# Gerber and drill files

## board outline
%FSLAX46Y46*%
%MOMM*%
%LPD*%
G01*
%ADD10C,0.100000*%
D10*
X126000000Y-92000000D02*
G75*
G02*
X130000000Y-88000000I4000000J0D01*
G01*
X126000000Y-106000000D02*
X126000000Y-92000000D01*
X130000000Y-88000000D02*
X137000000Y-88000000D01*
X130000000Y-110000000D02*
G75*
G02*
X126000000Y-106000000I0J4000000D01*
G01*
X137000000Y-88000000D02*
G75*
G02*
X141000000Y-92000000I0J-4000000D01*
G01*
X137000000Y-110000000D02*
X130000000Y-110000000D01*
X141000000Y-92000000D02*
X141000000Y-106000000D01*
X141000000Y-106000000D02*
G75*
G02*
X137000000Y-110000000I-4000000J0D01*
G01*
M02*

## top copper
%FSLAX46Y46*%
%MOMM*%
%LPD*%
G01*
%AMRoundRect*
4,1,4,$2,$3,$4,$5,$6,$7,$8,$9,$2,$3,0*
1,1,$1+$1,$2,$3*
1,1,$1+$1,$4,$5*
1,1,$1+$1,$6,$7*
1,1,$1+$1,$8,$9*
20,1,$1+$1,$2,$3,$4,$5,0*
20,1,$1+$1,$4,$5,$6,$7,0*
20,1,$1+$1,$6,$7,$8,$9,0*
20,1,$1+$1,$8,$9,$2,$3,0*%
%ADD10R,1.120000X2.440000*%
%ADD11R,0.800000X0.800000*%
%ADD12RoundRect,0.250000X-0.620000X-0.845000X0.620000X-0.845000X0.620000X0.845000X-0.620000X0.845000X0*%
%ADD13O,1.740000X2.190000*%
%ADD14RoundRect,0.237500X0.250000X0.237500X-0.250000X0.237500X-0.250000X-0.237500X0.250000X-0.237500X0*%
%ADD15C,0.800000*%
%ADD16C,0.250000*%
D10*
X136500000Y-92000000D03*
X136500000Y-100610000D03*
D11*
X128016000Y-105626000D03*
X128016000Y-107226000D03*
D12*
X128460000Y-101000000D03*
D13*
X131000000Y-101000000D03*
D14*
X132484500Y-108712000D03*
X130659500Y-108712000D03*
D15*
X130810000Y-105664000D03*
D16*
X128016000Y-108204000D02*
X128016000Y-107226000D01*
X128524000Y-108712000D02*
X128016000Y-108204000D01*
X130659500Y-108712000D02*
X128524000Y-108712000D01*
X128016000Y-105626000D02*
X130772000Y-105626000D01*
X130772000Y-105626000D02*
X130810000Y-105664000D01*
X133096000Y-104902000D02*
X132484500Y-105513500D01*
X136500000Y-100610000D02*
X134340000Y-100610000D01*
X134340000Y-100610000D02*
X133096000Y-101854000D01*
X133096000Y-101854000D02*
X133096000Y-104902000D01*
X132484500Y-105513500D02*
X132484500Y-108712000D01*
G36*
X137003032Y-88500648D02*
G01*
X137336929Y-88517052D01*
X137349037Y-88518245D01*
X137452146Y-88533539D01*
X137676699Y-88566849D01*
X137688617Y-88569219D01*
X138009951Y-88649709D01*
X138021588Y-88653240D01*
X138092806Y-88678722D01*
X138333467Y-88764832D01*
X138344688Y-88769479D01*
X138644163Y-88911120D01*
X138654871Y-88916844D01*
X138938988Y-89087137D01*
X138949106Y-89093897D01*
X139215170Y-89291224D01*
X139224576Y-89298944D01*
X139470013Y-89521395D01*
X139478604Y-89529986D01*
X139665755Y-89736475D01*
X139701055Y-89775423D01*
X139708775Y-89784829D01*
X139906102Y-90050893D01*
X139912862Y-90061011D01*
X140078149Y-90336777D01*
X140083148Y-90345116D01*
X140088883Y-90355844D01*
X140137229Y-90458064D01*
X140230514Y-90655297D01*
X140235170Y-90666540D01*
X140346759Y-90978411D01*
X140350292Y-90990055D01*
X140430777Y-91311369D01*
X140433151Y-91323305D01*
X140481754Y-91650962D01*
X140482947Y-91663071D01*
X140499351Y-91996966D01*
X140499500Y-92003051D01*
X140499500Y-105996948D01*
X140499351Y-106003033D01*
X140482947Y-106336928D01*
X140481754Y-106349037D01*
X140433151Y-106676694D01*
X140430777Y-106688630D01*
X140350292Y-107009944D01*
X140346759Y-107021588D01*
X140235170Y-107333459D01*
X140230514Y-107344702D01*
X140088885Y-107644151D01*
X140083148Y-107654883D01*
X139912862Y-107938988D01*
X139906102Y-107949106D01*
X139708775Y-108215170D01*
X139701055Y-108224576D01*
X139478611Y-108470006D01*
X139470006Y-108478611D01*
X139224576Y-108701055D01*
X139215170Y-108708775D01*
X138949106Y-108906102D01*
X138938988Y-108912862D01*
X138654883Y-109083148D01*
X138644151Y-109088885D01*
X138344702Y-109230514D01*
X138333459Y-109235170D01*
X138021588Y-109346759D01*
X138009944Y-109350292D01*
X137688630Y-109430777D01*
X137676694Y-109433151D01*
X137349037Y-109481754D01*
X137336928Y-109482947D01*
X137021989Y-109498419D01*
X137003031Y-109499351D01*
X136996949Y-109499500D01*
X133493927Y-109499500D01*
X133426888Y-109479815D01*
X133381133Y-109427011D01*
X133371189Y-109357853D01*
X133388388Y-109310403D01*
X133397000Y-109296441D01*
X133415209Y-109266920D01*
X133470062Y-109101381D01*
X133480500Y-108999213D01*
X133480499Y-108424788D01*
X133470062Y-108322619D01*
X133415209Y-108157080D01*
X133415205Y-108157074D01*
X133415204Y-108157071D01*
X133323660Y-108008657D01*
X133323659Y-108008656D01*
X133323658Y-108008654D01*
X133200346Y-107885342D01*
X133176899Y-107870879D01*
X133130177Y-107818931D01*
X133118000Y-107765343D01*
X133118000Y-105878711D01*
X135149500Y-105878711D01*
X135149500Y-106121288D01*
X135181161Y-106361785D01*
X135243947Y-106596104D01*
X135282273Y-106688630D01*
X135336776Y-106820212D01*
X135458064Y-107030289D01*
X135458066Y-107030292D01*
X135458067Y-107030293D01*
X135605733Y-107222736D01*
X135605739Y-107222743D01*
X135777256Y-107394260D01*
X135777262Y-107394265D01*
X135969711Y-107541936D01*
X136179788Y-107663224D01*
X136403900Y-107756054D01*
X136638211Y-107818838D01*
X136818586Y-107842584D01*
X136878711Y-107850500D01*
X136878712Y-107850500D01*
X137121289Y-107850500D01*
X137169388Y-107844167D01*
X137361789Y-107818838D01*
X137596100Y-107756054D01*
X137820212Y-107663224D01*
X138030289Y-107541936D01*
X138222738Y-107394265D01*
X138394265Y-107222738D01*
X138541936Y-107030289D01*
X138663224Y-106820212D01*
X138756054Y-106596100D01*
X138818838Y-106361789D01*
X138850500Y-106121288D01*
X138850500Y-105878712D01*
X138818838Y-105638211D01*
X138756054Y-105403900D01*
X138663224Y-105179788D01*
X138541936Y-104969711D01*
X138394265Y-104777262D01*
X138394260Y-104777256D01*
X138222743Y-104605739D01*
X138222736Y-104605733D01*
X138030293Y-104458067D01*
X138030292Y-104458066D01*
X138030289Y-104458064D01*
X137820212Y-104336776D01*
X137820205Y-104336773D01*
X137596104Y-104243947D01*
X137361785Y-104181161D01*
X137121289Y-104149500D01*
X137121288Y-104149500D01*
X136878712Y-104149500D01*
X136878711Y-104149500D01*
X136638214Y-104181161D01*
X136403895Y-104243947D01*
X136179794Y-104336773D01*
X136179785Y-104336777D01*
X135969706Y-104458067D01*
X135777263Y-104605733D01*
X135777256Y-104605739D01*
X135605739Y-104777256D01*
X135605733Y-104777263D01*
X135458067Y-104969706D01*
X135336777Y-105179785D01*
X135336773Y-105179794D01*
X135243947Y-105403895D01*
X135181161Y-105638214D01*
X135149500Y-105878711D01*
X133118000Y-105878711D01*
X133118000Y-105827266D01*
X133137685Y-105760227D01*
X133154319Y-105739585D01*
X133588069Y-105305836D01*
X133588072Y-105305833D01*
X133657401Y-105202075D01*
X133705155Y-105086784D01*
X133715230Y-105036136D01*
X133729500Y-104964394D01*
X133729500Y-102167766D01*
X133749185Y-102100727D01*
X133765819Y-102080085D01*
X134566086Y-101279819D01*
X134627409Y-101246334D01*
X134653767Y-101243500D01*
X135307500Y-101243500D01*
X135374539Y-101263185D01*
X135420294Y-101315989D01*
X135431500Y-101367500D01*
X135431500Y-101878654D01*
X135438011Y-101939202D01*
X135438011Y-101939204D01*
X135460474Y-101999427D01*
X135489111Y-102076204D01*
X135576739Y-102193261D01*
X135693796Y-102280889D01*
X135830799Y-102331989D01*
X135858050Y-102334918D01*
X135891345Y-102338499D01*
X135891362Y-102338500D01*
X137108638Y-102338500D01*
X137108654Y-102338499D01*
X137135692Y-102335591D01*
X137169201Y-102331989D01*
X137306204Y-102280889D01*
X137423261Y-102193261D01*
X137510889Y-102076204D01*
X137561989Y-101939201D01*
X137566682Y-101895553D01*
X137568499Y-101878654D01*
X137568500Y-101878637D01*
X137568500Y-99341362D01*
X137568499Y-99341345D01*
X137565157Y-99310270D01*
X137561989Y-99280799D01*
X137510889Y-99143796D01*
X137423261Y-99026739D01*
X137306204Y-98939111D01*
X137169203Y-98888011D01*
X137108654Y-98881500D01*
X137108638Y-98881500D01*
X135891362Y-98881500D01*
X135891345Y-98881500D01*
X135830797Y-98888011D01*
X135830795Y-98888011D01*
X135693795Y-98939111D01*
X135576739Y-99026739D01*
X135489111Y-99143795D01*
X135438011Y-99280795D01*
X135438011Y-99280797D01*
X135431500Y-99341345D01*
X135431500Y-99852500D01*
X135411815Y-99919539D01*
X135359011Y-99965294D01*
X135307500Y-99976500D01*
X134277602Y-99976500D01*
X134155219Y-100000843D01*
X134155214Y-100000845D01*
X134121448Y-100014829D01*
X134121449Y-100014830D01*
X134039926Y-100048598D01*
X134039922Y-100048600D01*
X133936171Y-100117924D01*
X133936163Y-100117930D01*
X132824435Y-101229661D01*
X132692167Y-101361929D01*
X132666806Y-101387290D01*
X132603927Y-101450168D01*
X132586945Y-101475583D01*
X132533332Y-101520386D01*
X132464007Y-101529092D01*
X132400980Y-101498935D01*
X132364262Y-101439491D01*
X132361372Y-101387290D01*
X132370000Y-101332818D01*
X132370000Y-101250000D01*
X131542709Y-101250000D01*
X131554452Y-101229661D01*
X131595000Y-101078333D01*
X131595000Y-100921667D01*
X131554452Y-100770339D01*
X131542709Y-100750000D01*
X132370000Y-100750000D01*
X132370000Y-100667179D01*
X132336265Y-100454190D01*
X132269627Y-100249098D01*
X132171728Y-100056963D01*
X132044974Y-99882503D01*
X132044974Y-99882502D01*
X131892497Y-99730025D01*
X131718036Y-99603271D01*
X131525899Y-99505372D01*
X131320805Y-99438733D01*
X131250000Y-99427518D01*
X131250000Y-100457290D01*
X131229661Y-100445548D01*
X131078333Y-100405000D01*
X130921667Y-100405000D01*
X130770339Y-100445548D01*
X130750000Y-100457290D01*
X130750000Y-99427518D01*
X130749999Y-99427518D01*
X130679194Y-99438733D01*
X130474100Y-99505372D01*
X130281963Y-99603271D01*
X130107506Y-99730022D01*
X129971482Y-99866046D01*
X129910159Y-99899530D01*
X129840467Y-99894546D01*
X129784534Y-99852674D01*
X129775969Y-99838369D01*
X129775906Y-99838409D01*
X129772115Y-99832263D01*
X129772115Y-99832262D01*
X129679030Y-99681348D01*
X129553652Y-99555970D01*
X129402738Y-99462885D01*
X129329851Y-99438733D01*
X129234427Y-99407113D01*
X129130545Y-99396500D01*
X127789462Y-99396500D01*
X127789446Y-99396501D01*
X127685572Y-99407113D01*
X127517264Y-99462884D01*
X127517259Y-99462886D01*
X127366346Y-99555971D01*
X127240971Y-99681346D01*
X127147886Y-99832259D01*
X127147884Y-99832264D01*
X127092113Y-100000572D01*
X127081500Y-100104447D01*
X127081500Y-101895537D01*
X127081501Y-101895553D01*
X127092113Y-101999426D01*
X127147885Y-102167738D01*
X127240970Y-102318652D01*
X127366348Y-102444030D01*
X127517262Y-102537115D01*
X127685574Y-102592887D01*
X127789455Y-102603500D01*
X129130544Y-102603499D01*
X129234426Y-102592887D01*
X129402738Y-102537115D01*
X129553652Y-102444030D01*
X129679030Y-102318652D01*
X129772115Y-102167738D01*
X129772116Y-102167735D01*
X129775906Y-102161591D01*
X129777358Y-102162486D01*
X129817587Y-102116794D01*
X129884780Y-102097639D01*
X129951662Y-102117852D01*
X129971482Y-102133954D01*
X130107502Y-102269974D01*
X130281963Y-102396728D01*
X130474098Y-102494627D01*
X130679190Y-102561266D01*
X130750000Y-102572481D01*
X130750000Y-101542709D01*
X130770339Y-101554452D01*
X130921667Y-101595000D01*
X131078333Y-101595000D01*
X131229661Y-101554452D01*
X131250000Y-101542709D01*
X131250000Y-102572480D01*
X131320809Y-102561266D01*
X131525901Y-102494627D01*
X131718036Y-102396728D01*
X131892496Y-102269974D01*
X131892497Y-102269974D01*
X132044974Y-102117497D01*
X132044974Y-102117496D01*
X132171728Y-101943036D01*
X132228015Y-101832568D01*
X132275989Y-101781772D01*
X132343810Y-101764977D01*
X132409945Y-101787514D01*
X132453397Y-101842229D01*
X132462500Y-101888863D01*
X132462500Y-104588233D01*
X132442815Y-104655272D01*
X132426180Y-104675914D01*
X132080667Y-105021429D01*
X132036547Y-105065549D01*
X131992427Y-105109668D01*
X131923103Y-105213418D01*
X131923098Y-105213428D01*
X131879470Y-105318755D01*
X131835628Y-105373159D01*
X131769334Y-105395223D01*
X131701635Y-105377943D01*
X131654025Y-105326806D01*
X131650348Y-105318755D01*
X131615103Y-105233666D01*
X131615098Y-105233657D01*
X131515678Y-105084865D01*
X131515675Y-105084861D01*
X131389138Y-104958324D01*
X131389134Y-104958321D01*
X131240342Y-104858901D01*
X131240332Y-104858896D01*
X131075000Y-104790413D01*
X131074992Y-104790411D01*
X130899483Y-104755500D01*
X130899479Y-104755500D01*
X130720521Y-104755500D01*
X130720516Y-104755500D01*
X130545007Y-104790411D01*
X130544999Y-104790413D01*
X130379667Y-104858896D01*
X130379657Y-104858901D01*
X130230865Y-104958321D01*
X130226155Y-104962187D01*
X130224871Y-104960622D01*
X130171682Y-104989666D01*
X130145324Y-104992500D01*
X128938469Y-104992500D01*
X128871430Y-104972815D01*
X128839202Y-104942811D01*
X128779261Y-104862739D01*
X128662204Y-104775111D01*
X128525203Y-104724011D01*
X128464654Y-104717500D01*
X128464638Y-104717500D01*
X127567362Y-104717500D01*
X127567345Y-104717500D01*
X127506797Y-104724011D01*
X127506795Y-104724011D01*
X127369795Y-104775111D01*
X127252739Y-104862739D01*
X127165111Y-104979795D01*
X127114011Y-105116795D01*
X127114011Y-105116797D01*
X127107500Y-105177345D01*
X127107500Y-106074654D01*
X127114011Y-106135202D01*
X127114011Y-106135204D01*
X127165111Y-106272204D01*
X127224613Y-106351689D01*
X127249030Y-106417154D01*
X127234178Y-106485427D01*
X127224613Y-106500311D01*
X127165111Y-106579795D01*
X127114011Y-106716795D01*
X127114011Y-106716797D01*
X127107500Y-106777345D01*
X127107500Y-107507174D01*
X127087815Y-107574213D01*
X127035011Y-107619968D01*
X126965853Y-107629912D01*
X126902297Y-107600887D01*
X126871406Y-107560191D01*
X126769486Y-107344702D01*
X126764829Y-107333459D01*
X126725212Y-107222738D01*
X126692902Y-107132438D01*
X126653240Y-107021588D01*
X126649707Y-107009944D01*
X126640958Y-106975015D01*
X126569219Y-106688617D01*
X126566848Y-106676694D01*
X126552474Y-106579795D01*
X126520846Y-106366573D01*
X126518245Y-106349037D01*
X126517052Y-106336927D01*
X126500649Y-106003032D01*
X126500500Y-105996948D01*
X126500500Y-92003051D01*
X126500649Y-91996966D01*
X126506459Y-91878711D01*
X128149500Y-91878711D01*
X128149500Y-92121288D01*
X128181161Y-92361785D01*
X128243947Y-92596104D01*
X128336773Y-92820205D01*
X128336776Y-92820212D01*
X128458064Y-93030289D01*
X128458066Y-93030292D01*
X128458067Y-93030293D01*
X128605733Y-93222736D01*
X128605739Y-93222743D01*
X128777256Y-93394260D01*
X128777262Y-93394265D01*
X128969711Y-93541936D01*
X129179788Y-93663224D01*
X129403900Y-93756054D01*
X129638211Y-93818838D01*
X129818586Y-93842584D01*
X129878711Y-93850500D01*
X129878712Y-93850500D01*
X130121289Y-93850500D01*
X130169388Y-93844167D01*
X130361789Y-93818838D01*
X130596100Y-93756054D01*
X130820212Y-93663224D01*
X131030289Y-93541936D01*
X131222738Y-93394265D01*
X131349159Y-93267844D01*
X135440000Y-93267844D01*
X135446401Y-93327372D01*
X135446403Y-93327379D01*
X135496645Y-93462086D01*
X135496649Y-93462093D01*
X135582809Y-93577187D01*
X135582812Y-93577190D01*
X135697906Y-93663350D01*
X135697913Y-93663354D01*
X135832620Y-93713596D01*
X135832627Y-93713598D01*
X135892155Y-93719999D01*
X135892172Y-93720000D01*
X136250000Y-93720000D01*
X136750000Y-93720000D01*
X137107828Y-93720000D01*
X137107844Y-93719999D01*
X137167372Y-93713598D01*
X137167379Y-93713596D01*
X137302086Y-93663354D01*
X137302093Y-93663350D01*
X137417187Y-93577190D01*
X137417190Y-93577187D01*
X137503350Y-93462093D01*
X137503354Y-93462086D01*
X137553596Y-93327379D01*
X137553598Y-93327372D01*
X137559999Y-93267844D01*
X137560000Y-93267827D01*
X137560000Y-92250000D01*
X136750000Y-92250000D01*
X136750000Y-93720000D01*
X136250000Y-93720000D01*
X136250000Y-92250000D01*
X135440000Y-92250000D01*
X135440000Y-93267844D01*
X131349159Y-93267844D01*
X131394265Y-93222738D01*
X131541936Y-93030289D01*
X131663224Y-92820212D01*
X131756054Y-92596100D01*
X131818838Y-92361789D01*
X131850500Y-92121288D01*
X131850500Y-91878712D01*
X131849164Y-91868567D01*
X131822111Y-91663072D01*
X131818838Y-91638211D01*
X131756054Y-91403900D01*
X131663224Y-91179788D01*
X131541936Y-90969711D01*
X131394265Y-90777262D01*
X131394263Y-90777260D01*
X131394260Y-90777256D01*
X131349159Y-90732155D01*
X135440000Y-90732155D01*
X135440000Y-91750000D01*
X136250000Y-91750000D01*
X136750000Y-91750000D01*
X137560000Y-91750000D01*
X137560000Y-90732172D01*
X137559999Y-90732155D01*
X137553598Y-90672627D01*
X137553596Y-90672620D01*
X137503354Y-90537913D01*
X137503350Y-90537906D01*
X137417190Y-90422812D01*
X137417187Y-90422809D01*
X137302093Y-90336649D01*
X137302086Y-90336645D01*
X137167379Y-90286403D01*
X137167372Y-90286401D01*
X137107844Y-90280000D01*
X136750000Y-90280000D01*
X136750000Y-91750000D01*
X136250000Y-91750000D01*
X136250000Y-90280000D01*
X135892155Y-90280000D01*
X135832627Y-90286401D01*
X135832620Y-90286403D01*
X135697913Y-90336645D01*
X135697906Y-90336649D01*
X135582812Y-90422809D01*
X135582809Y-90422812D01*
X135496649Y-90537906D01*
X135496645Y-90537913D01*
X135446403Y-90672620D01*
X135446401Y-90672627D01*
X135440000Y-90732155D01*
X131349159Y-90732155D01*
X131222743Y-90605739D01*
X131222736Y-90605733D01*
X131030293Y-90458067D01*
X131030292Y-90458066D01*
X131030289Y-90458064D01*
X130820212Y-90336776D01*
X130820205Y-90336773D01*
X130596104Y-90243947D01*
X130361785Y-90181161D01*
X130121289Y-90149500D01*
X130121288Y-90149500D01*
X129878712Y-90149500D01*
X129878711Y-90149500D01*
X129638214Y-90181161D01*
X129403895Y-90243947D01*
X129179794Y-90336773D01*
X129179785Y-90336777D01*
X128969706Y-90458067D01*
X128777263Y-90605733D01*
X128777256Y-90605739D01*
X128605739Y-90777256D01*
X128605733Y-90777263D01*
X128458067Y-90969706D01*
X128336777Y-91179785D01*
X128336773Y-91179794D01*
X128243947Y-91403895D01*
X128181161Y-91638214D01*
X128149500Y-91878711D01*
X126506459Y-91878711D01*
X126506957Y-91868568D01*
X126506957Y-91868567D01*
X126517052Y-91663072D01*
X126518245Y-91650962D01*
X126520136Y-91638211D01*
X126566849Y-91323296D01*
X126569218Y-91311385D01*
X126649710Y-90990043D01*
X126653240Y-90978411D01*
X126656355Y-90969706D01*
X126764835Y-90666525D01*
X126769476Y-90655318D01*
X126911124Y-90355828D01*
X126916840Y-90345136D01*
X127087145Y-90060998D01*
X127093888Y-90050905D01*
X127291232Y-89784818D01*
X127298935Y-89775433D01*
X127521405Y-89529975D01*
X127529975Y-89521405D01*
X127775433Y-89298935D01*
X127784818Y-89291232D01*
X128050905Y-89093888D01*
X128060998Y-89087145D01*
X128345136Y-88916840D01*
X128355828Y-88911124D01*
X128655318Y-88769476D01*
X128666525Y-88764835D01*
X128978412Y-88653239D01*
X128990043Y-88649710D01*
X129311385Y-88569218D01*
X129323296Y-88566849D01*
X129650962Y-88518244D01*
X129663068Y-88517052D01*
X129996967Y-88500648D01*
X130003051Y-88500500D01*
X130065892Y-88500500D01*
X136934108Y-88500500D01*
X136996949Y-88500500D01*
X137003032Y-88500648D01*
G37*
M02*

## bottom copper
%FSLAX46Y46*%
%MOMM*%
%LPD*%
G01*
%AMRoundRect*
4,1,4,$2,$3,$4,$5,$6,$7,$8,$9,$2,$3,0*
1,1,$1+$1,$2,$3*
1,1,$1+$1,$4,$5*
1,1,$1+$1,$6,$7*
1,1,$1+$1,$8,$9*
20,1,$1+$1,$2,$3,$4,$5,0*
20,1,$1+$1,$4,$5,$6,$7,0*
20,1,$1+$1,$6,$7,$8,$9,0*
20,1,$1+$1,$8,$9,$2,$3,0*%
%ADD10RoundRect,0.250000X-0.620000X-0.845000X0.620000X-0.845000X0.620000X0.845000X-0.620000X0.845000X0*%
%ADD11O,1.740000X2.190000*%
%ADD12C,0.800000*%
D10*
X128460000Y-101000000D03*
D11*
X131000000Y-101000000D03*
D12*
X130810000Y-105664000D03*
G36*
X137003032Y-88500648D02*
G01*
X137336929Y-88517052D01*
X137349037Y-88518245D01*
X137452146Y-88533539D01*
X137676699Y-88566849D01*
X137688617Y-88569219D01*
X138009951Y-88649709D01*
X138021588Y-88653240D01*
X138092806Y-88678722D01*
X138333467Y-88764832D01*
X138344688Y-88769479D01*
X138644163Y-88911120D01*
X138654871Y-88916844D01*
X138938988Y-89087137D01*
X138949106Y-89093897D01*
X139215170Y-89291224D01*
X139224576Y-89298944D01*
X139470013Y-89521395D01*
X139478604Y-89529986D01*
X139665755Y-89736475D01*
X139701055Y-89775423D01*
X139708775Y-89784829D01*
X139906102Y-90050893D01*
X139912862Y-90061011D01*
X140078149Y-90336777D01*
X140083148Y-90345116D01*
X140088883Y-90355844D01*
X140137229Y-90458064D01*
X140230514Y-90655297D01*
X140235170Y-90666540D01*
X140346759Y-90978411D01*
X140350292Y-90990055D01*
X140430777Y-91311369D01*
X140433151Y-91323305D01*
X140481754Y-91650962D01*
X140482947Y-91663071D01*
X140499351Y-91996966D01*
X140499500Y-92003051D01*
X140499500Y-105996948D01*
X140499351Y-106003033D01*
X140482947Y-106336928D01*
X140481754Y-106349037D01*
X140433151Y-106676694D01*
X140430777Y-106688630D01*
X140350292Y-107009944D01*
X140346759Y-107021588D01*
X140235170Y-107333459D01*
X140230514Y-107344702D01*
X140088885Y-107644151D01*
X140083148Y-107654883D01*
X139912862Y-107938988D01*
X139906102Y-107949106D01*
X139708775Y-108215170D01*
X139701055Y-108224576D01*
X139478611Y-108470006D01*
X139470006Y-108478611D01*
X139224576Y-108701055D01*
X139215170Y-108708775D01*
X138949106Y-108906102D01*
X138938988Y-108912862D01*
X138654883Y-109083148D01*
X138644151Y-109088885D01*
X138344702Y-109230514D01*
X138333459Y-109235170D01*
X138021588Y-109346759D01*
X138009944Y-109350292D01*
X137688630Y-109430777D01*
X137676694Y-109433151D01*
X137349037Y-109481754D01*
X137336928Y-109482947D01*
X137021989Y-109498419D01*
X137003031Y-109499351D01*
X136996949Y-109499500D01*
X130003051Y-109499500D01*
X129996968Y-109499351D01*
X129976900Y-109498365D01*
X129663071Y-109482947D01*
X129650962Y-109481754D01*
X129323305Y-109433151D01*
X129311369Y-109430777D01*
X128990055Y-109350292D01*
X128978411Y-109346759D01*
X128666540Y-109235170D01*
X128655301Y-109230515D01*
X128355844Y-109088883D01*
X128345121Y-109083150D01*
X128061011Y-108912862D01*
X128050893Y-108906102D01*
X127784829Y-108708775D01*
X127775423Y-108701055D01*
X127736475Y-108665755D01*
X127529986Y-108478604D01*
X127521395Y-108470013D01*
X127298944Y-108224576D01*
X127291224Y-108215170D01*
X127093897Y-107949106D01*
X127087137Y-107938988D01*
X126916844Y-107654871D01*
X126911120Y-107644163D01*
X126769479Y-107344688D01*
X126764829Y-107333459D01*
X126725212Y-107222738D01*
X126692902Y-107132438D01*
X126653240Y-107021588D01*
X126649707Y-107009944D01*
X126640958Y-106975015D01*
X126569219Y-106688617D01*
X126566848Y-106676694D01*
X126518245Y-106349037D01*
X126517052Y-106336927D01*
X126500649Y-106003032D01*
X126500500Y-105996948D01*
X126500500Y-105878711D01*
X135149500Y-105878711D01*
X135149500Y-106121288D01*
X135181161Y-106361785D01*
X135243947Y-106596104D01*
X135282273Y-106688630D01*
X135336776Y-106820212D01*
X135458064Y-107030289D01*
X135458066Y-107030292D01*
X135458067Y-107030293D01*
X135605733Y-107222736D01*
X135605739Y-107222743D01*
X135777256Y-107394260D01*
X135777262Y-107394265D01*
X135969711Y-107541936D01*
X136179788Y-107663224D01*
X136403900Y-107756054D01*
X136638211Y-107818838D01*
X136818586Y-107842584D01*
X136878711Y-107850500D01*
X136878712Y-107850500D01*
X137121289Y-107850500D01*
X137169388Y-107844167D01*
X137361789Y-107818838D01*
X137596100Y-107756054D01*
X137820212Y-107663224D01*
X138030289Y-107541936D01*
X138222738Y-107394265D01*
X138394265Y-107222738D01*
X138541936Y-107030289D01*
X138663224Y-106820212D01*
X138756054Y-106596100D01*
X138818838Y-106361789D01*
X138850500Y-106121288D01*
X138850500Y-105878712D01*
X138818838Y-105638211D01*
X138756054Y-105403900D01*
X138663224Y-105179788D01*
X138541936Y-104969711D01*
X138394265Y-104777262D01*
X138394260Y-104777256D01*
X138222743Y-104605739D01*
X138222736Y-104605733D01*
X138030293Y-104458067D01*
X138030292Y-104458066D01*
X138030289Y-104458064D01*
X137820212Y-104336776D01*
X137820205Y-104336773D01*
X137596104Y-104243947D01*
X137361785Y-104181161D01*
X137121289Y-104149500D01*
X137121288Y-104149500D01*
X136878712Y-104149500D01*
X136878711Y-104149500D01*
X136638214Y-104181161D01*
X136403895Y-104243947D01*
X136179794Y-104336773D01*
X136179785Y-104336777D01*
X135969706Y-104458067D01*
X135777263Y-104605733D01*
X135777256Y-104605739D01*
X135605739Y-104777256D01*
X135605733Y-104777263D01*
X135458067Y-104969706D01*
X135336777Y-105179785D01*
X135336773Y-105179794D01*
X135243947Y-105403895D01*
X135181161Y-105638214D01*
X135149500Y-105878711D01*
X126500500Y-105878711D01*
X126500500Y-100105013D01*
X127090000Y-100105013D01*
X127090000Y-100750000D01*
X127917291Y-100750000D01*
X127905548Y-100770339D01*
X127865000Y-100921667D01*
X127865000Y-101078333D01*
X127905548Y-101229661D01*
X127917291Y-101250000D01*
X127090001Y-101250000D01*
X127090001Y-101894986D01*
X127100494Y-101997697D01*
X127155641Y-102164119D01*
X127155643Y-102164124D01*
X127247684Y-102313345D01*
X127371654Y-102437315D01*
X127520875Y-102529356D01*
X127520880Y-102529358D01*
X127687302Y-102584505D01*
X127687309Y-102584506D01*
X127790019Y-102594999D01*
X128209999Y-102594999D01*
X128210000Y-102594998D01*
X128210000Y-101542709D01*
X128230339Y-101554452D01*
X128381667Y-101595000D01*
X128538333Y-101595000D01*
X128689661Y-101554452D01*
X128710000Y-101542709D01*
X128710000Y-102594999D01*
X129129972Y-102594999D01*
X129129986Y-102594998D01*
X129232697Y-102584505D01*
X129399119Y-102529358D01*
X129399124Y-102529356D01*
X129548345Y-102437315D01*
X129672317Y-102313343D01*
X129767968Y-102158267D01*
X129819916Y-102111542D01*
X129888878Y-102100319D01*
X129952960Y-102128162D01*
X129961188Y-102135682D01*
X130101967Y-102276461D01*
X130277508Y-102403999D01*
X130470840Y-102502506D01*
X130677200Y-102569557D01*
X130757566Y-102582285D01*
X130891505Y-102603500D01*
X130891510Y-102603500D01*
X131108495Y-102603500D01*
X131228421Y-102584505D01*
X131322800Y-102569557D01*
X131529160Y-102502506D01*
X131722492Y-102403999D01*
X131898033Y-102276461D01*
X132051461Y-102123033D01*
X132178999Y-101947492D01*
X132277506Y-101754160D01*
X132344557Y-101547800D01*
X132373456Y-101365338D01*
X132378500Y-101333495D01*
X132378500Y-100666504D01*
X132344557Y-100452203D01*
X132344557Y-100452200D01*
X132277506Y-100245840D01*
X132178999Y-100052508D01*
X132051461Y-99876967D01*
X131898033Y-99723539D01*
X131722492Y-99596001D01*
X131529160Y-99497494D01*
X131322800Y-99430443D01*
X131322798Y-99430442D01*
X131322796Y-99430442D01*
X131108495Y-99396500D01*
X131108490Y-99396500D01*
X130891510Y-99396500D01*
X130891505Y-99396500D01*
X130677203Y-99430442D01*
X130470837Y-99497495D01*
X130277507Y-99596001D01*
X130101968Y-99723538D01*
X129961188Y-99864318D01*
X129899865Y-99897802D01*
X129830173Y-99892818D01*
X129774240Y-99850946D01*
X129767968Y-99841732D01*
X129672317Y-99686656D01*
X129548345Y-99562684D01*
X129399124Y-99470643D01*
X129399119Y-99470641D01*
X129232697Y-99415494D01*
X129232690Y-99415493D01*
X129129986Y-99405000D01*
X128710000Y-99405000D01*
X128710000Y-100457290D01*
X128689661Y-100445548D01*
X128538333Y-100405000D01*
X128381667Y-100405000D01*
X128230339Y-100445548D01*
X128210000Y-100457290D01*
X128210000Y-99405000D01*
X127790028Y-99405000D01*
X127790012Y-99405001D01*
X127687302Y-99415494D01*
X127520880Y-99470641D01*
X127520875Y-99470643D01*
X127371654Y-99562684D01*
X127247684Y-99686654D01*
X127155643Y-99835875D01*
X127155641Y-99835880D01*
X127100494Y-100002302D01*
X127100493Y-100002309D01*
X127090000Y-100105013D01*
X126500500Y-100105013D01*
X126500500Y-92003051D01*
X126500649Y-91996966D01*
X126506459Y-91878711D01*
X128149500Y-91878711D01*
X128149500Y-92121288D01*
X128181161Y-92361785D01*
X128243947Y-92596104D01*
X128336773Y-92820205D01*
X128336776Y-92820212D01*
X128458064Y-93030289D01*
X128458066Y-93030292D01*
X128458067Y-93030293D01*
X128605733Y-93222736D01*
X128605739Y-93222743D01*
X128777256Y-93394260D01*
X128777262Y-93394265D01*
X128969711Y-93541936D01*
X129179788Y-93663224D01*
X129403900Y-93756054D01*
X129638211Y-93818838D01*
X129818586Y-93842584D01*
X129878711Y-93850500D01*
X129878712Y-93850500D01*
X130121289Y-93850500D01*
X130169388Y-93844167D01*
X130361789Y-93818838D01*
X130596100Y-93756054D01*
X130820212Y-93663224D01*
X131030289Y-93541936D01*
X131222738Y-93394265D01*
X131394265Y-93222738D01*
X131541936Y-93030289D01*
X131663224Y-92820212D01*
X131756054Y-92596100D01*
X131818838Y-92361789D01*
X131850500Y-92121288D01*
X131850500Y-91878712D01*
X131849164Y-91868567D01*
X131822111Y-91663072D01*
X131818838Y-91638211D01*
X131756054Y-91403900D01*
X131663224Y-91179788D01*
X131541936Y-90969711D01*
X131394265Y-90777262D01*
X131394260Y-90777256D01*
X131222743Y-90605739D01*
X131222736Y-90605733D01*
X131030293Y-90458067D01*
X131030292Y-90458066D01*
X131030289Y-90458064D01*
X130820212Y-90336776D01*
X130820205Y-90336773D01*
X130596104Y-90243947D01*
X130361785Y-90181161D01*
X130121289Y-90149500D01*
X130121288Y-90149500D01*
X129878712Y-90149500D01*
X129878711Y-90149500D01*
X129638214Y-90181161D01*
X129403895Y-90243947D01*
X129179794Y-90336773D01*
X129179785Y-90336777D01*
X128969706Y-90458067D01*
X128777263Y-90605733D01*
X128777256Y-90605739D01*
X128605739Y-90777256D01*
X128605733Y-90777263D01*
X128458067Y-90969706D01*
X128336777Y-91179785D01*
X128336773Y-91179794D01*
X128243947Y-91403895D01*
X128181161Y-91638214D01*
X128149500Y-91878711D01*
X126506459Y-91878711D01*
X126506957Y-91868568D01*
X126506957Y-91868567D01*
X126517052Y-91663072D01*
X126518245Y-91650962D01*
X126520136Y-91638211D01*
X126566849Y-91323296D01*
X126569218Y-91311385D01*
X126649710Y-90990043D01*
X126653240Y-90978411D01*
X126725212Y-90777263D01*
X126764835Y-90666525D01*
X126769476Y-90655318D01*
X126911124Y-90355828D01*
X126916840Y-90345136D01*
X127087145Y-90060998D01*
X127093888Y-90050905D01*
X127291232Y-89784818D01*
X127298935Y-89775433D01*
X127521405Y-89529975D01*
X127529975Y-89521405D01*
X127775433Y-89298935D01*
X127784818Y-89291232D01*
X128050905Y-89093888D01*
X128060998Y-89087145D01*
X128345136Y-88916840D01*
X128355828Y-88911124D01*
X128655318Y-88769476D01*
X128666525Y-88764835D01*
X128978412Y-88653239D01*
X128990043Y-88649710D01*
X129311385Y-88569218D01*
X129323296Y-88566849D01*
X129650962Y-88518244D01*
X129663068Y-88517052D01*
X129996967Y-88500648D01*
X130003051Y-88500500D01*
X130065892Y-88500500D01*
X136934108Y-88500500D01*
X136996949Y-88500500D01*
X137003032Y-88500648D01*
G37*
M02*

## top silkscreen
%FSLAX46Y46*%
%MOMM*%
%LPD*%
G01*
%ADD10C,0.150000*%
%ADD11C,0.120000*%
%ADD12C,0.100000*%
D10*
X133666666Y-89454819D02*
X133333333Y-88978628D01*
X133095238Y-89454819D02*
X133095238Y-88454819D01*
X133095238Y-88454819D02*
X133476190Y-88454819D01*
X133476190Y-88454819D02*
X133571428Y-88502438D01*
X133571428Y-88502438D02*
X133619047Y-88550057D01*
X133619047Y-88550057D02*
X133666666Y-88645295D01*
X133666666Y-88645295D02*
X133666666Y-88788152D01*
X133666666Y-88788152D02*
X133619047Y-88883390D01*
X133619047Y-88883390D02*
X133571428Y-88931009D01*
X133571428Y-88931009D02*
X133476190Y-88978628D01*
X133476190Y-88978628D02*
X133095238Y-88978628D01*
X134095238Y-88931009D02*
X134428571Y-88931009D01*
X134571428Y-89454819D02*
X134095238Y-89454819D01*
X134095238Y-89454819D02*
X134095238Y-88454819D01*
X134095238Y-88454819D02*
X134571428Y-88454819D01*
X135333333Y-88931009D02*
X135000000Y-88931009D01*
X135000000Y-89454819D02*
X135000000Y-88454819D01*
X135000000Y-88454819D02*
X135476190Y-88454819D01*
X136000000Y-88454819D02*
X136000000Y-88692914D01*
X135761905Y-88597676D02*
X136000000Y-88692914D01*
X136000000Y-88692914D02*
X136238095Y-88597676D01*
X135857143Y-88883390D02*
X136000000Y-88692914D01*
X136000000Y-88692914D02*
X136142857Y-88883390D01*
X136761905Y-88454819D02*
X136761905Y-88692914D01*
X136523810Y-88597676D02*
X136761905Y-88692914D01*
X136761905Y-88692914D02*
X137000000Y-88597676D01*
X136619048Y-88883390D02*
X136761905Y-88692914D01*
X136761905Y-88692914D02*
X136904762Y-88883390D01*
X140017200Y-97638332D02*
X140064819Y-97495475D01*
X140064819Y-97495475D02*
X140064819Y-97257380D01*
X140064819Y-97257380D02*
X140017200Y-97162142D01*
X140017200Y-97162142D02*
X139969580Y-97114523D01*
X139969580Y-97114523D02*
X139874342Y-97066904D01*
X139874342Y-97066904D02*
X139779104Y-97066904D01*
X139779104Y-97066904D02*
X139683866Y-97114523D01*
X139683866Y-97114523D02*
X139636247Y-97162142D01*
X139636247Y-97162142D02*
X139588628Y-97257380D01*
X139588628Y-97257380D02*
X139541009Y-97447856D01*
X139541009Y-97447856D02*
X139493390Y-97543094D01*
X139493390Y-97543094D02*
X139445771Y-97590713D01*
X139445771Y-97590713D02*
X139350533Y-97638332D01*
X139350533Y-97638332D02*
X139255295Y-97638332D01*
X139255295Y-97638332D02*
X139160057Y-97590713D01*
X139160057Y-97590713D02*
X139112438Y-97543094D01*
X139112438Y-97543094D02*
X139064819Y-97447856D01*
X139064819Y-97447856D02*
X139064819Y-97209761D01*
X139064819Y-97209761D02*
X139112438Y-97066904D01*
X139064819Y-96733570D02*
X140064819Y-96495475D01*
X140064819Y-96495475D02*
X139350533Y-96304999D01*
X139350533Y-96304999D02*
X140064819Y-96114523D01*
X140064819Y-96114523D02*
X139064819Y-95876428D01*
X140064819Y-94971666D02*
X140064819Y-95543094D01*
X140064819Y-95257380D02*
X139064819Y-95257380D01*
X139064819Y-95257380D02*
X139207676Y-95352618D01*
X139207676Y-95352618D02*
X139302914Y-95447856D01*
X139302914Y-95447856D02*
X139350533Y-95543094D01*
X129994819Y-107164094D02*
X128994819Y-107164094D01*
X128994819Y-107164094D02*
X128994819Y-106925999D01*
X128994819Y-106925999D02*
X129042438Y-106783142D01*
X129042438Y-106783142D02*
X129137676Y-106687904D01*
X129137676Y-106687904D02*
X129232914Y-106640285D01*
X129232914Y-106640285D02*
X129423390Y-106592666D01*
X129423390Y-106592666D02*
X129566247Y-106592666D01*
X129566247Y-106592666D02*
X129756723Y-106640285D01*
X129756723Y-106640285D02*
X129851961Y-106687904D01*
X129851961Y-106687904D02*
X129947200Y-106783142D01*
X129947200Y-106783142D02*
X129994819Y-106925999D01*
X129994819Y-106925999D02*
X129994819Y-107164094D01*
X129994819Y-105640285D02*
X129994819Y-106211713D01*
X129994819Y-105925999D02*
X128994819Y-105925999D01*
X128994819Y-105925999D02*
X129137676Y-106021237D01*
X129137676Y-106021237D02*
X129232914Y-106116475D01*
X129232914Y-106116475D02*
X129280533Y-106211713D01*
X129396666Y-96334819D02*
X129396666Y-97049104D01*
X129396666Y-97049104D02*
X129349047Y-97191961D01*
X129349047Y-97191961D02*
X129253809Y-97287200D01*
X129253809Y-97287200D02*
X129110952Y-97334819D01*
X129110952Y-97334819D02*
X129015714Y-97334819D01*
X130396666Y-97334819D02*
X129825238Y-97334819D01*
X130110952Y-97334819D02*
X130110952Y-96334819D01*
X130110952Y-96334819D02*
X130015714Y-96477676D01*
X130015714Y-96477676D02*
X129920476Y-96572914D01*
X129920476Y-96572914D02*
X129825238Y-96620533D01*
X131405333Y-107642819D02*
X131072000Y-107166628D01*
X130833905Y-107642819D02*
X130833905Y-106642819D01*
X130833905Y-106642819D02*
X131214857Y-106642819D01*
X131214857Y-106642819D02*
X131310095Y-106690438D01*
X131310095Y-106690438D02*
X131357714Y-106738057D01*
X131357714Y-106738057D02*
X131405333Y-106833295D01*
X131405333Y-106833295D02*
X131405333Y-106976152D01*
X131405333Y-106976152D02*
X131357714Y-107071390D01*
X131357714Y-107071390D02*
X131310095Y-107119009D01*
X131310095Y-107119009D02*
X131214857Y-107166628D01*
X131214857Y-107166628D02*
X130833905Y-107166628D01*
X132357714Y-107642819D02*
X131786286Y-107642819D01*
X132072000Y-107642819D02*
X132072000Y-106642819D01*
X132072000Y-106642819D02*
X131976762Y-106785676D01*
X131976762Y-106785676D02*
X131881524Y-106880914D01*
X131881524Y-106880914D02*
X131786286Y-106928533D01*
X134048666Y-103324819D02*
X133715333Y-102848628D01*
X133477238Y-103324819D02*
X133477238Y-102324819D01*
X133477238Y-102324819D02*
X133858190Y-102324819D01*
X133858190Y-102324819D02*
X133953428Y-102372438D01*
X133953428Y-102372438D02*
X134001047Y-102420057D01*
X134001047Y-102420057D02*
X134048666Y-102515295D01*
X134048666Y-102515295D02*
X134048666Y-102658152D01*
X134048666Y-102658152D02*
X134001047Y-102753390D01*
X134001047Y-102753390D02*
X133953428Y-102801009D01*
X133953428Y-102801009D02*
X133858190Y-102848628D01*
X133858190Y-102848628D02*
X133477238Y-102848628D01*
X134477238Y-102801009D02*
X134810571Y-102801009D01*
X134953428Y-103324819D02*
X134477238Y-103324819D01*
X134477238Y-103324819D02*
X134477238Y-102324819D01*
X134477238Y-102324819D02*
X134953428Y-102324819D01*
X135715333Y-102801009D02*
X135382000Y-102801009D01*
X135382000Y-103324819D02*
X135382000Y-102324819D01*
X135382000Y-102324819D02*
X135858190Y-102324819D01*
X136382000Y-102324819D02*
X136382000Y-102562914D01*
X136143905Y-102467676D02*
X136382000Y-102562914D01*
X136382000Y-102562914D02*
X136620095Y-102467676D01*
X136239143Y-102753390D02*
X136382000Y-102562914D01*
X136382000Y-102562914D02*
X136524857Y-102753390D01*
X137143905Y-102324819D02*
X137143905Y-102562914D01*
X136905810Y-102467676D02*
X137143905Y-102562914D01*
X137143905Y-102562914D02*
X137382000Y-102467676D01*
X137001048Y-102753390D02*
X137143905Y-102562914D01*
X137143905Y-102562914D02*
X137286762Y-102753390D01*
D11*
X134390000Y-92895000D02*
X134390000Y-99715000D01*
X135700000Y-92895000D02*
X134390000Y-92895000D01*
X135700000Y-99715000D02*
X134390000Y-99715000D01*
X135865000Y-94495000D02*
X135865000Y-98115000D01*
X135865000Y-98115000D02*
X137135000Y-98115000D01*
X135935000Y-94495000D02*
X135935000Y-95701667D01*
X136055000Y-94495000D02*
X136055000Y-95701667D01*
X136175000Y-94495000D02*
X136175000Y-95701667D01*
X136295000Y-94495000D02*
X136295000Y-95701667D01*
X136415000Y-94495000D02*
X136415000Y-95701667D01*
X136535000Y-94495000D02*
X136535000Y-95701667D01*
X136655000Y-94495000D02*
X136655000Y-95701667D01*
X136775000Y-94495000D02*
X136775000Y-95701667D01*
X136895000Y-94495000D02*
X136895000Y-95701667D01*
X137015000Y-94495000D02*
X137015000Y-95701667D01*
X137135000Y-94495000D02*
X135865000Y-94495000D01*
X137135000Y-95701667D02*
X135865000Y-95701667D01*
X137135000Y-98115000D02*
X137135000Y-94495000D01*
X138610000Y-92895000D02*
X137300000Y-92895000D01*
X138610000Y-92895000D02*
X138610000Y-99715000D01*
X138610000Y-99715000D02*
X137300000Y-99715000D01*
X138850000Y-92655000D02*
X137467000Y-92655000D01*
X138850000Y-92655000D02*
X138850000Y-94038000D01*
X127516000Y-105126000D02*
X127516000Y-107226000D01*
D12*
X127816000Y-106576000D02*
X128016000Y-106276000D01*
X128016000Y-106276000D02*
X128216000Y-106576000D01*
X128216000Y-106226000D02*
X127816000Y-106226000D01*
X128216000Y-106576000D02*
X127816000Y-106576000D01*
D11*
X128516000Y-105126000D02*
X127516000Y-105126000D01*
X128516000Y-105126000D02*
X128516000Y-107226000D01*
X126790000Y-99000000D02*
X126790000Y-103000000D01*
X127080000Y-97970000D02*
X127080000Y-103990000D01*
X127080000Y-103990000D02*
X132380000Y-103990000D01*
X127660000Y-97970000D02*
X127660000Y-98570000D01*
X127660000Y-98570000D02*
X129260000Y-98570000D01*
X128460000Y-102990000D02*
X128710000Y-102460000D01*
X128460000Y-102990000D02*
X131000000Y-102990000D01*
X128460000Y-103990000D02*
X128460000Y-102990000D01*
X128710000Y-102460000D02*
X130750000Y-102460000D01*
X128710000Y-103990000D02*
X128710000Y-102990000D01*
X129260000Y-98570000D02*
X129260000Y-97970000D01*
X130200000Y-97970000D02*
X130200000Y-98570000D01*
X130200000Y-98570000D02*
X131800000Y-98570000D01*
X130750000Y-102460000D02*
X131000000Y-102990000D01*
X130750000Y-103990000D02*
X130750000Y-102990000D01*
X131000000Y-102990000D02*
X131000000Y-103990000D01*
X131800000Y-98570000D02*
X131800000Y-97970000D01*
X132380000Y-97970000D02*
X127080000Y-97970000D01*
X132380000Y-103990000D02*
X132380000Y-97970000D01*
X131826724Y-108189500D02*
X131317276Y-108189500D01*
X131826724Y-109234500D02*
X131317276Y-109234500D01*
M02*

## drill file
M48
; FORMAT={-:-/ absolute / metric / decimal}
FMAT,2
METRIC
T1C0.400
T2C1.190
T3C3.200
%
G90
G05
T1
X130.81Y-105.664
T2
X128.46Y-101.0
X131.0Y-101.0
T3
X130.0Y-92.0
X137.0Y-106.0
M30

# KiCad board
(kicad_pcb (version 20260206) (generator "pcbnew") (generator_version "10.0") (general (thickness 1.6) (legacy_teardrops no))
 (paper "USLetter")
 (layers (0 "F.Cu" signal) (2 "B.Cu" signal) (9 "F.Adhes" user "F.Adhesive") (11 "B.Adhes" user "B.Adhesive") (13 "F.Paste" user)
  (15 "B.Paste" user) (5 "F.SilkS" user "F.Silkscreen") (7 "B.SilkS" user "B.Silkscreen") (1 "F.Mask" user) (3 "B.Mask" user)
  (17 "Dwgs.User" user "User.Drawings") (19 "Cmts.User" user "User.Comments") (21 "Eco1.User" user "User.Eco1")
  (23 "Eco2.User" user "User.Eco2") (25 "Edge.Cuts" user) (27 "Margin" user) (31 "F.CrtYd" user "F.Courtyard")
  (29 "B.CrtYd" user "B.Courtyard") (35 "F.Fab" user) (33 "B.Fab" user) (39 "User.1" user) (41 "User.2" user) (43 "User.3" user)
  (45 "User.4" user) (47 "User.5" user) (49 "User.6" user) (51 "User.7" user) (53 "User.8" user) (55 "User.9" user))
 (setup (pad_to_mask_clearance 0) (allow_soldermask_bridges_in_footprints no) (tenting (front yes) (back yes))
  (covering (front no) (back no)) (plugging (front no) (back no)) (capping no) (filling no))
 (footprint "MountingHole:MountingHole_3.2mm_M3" (layer "F.Cu") (at 130 92)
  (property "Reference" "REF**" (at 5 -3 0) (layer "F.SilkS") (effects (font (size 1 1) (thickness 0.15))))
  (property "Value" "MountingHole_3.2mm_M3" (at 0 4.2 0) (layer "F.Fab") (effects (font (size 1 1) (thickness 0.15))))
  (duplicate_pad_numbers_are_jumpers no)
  (pad "" np_thru_hole circle (at 0 0) (size 3.2 3.2) (drill 3.2) (layers "*.Cu" "*.Mask")))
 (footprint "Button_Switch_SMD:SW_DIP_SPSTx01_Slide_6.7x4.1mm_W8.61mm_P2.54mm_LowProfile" (layer "F.Cu") (at 136.5 96.305 -90)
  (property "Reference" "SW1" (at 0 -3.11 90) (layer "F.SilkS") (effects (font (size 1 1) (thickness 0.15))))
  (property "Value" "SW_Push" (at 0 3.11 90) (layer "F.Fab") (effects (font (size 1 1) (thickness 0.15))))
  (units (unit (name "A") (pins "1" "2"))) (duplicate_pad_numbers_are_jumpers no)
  (fp_line (start -3.41 2.11) (end 3.41 2.11) (stroke (width 0.12) (type solid)) (layer "F.SilkS"))
  (fp_line (start -3.41 0.8) (end -3.41 2.11) (stroke (width 0.12) (type solid)) (layer "F.SilkS"))
  (fp_line (start 3.41 0.8) (end 3.41 2.11) (stroke (width 0.12) (type solid)) (layer "F.SilkS"))
  (fp_line (start -1.81 0.635) (end 1.81 0.635) (stroke (width 0.12) (type solid)) (layer "F.SilkS"))
  (fp_line (start 1.81 0.635) (end 1.81 -0.635) (stroke (width 0.12) (type solid)) (layer "F.SilkS"))
  (fp_line (start -1.81 0.565) (end -0.603333 0.565) (stroke (width 0.12) (type solid)) (layer "F.SilkS"))
  (fp_line (start -1.81 0.445) (end -0.603333 0.445) (stroke (width 0.12) (type solid)) (layer "F.SilkS"))
  (fp_line (start -1.81 0.325) (end -0.603333 0.325) (stroke (width 0.12) (type solid)) (layer "F.SilkS"))
  (fp_line (start -1.81 0.205) (end -0.603333 0.205) (stroke (width 0.12) (type solid)) (layer "F.SilkS"))
  (fp_line (start -1.81 0.085) (end -0.603333 0.085) (stroke (width 0.12) (type solid)) (layer "F.SilkS"))
  (fp_line (start -1.81 -0.035) (end -0.603333 -0.035) (stroke (width 0.12) (type solid)) (layer "F.SilkS"))
  (fp_line (start -1.81 -0.155) (end -0.603333 -0.155) (stroke (width 0.12) (type solid)) (layer "F.SilkS"))
  (fp_line (start -1.81 -0.275) (end -0.603333 -0.275) (stroke (width 0.12) (type solid)) (layer "F.SilkS"))
  (fp_line (start -1.81 -0.395) (end -0.603333 -0.395) (stroke (width 0.12) (type solid)) (layer "F.SilkS"))
  (fp_line (start -1.81 -0.515) (end -0.603333 -0.515) (stroke (width 0.12) (type solid)) (layer "F.SilkS"))
  (fp_line (start -1.81 -0.635) (end -1.81 0.635) (stroke (width 0.12) (type solid)) (layer "F.SilkS"))
  (fp_line (start -0.603333 -0.635) (end -0.603333 0.635) (stroke (width 0.12) (type solid)) (layer "F.SilkS"))
  (fp_line (start 1.81 -0.635) (end -1.81 -0.635) (stroke (width 0.12) (type solid)) (layer "F.SilkS"))
  (fp_line (start -3.41 -2.11) (end -3.41 -0.8) (stroke (width 0.12) (type solid)) (layer "F.SilkS"))
  (fp_line (start -3.41 -2.11) (end 3.41 -2.11) (stroke (width 0.12) (type solid)) (layer "F.SilkS"))
  (fp_line (start 3.41 -2.11) (end 3.41 -0.8) (stroke (width 0.12) (type solid)) (layer "F.SilkS"))
  (fp_line (start -3.65 -2.35) (end -3.65 -0.967) (stroke (width 0.12) (type solid)) (layer "F.SilkS"))
  (fp_line (start -3.65 -2.35) (end -2.267 -2.35) (stroke (width 0.12) (type solid)) (layer "F.SilkS"))
  (pad "1" smd rect (at -4.305 0 270) (size 2.44 1.12) (layers "F.Cu" "F.Mask" "F.Paste") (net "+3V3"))
  (pad "2" smd rect (at 4.305 0 270) (size 2.44 1.12) (layers "F.Cu" "F.Mask" "F.Paste") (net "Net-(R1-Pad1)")))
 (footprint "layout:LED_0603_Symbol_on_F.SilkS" (layer "F.Cu") (at 128.016 106.426 -90)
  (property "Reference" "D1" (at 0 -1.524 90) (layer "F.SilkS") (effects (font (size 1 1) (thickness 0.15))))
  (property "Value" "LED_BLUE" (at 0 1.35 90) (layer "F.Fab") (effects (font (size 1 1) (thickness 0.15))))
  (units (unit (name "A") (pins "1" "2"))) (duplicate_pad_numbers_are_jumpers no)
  (fp_line (start -1.3 0.5) (end 0.8 0.5) (stroke (width 0.12) (type solid)) (layer "F.SilkS"))
  (fp_line (start 0.15 0.2) (end -0.15 0) (stroke (width 0.1) (type solid)) (layer "F.SilkS"))
  (fp_line (start -0.15 0) (end 0.15 -0.2) (stroke (width 0.1) (type solid)) (layer "F.SilkS"))
  (fp_line (start -0.2 -0.2) (end -0.2 0.2) (stroke (width 0.1) (type solid)) (layer "F.SilkS"))
  (fp_line (start 0.15 -0.2) (end 0.15 0.2) (stroke (width 0.1) (type solid)) (layer "F.SilkS"))
  (fp_line (start -1.3 -0.5) (end -1.3 0.5) (stroke (width 0.12) (type solid)) (layer "F.SilkS"))
  (fp_line (start -1.3 -0.5) (end 0.8 -0.5) (stroke (width 0.12) (type solid)) (layer "F.SilkS"))
  (pad "1" smd rect (at -0.8 0 90) (size 0.8 0.8) (layers "F.Cu" "F.Mask" "F.Paste") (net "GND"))
  (pad "2" smd rect (at 0.8 0 90) (size 0.8 0.8) (layers "F.Cu" "F.Mask" "F.Paste") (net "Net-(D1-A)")))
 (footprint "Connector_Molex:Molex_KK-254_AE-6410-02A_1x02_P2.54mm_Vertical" (layer "F.Cu") (at 128.46 101)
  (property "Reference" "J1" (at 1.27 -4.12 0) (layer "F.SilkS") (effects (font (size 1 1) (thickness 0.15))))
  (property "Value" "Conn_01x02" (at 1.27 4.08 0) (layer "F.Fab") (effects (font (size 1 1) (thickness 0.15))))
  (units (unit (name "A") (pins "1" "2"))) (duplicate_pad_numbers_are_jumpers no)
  (fp_line (start -1.67 -2) (end -1.67 2) (stroke (width 0.12) (type solid)) (layer "F.SilkS"))
  (fp_line (start -1.38 -3.03) (end -1.38 2.99) (stroke (width 0.12) (type solid)) (layer "F.SilkS"))
  (fp_line (start -1.38 2.99) (end 3.92 2.99) (stroke (width 0.12) (type solid)) (layer "F.SilkS"))
  (fp_line (start -0.8 -3.03) (end -0.8 -2.43) (stroke (width 0.12) (type solid)) (layer "F.SilkS"))
  (fp_line (start -0.8 -2.43) (end 0.8 -2.43) (stroke (width 0.12) (type solid)) (layer "F.SilkS"))
  (fp_line (start 0 1.99) (end 0.25 1.46) (stroke (width 0.12) (type solid)) (layer "F.SilkS"))
  (fp_line (start 0 1.99) (end 2.54 1.99) (stroke (width 0.12) (type solid)) (layer "F.SilkS"))
  (fp_line (start 0 2.99) (end 0 1.99) (stroke (width 0.12) (type solid)) (layer "F.SilkS"))
  (fp_line (start 0.25 1.46) (end 2.29 1.46) (stroke (width 0.12) (type solid)) (layer "F.SilkS"))
  (fp_line (start 0.25 2.99) (end 0.25 1.99) (stroke (width 0.12) (type solid)) (layer "F.SilkS"))
  (fp_line (start 0.8 -2.43) (end 0.8 -3.03) (stroke (width 0.12) (type solid)) (layer "F.SilkS"))
  (fp_line (start 1.74 -3.03) (end 1.74 -2.43) (stroke (width 0.12) (type solid)) (layer "F.SilkS"))
  (fp_line (start 1.74 -2.43) (end 3.34 -2.43) (stroke (width 0.12) (type solid)) (layer "F.SilkS"))
  (fp_line (start 2.29 1.46) (end 2.54 1.99) (stroke (width 0.12) (type solid)) (layer "F.SilkS"))
  (fp_line (start 2.29 2.99) (end 2.29 1.99) (stroke (width 0.12) (type solid)) (layer "F.SilkS"))
  (fp_line (start 2.54 1.99) (end 2.54 2.99) (stroke (width 0.12) (type solid)) (layer "F.SilkS"))
  (fp_line (start 3.34 -2.43) (end 3.34 -3.03) (stroke (width 0.12) (type solid)) (layer "F.SilkS"))
  (fp_line (start 3.92 -3.03) (end -1.38 -3.03) (stroke (width 0.12) (type solid)) (layer "F.SilkS"))
  (fp_line (start 3.92 2.99) (end 3.92 -3.03) (stroke (width 0.12) (type solid)) (layer "F.SilkS"))
  (pad "1" thru_hole roundrect (at 0 0) (size 1.74 2.19) (drill 1.19) (layers "*.Cu" "*.Mask") (remove_unused_layers no)
   (roundrect_rratio 0.143678) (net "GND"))
  (pad "2" thru_hole oval (at 2.54 0) (size 1.74 2.19) (drill 1.19) (layers "*.Cu" "*.Mask") (remove_unused_layers no) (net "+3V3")))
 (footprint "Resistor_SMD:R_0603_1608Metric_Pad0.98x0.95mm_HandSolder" (layer "F.Cu") (at 131.572 108.712 180)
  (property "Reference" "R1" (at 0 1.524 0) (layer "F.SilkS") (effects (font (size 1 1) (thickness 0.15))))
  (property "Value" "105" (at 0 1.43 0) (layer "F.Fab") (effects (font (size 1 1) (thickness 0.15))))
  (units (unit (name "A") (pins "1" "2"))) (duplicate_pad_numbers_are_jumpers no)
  (fp_line (start -0.254724 0.5225) (end 0.254724 0.5225) (stroke (width 0.12) (type solid)) (layer "F.SilkS"))
  (fp_line (start -0.254724 -0.5225) (end 0.254724 -0.5225) (stroke (width 0.12) (type solid)) (layer "F.SilkS"))
  (pad "1" smd roundrect (at -0.9125 0 180) (size 0.975 0.95) (layers "F.Cu" "F.Mask" "F.Paste") (roundrect_rratio 0.25)
   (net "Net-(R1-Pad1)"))
  (pad "2" smd roundrect (at 0.9125 0 180) (size 0.975 0.95) (layers "F.Cu" "F.Mask" "F.Paste") (roundrect_rratio 0.25) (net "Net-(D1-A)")))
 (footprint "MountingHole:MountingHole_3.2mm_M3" (layer "F.Cu") (at 137 106)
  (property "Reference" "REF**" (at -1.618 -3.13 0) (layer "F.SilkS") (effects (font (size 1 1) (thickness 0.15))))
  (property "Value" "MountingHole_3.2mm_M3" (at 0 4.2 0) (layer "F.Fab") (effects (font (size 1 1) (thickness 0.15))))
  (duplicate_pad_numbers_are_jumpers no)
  (pad "" np_thru_hole circle (at 0 0) (size 3.2 3.2) (drill 3.2) (layers "*.Cu" "*.Mask")))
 (gr_arc (start 126 92) (mid 127.171573 89.171573) (end 130 88) (stroke (width 0.1) (type default)) (layer "Edge.Cuts"))
 (gr_line (start 126 106) (end 126 92) (stroke (width 0.1) (type default)) (layer "Edge.Cuts"))
 (gr_line (start 130 88) (end 137 88) (stroke (width 0.1) (type default)) (layer "Edge.Cuts"))
 (gr_arc (start 130 110) (mid 127.171573 108.828427) (end 126 106) (stroke (width 0.1) (type default)) (layer "Edge.Cuts"))
 (gr_arc (start 137 88) (mid 139.828427 89.171573) (end 141 92) (stroke (width 0.1) (type default)) (layer "Edge.Cuts"))
 (gr_line (start 137 110) (end 130 110) (stroke (width 0.1) (type default)) (layer "Edge.Cuts"))
 (gr_line (start 141 92) (end 141 106) (stroke (width 0.1) (type default)) (layer "Edge.Cuts"))
 (gr_arc (start 141 106) (mid 139.828427 108.828427) (end 137 110) (stroke (width 0.1) (type default)) (layer "Edge.Cuts"))
 (segment (start 128.016 108.204) (end 128.016 107.226) (width 0.25) (layer "F.Cu") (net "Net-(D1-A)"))
 (segment (start 128.524 108.712) (end 128.016 108.204) (width 0.25) (layer "F.Cu") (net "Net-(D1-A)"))
 (segment (start 130.6595 108.712) (end 128.524 108.712) (width 0.25) (layer "F.Cu") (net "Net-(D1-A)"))
 (segment (start 128.016 105.626) (end 130.772 105.626) (width 0.25) (layer "F.Cu") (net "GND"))
 (segment (start 130.772 105.626) (end 130.81 105.664) (width 0.25) (layer "F.Cu") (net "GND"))
 (via (at 130.81 105.664) (size 0.8) (drill 0.4) (layers "F.Cu" "B.Cu") (free yes) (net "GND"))
 (segment (start 133.096 104.902) (end 132.4845 105.5135) (width 0.25) (layer "F.Cu") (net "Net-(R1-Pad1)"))
 (segment (start 136.5 100.61) (end 134.34 100.61) (width 0.25) (layer "F.Cu") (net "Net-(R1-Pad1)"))
 (segment (start 134.34 100.61) (end 133.096 101.854) (width 0.25) (layer "F.Cu") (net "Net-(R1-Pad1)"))
 (segment (start 133.096 101.854) (end 133.096 104.902) (width 0.25) (layer "F.Cu") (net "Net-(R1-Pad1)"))
 (segment (start 132.4845 105.5135) (end 132.4845 108.712) (width 0.25) (layer "F.Cu") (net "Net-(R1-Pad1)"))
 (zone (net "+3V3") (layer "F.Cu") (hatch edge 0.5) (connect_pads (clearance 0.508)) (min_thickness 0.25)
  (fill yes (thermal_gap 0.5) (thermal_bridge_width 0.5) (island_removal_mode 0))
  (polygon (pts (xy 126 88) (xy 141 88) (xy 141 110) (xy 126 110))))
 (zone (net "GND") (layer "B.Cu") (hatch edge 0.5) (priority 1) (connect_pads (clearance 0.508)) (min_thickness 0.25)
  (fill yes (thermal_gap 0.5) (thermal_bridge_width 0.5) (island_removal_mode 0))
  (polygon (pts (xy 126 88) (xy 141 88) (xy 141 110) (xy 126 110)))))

